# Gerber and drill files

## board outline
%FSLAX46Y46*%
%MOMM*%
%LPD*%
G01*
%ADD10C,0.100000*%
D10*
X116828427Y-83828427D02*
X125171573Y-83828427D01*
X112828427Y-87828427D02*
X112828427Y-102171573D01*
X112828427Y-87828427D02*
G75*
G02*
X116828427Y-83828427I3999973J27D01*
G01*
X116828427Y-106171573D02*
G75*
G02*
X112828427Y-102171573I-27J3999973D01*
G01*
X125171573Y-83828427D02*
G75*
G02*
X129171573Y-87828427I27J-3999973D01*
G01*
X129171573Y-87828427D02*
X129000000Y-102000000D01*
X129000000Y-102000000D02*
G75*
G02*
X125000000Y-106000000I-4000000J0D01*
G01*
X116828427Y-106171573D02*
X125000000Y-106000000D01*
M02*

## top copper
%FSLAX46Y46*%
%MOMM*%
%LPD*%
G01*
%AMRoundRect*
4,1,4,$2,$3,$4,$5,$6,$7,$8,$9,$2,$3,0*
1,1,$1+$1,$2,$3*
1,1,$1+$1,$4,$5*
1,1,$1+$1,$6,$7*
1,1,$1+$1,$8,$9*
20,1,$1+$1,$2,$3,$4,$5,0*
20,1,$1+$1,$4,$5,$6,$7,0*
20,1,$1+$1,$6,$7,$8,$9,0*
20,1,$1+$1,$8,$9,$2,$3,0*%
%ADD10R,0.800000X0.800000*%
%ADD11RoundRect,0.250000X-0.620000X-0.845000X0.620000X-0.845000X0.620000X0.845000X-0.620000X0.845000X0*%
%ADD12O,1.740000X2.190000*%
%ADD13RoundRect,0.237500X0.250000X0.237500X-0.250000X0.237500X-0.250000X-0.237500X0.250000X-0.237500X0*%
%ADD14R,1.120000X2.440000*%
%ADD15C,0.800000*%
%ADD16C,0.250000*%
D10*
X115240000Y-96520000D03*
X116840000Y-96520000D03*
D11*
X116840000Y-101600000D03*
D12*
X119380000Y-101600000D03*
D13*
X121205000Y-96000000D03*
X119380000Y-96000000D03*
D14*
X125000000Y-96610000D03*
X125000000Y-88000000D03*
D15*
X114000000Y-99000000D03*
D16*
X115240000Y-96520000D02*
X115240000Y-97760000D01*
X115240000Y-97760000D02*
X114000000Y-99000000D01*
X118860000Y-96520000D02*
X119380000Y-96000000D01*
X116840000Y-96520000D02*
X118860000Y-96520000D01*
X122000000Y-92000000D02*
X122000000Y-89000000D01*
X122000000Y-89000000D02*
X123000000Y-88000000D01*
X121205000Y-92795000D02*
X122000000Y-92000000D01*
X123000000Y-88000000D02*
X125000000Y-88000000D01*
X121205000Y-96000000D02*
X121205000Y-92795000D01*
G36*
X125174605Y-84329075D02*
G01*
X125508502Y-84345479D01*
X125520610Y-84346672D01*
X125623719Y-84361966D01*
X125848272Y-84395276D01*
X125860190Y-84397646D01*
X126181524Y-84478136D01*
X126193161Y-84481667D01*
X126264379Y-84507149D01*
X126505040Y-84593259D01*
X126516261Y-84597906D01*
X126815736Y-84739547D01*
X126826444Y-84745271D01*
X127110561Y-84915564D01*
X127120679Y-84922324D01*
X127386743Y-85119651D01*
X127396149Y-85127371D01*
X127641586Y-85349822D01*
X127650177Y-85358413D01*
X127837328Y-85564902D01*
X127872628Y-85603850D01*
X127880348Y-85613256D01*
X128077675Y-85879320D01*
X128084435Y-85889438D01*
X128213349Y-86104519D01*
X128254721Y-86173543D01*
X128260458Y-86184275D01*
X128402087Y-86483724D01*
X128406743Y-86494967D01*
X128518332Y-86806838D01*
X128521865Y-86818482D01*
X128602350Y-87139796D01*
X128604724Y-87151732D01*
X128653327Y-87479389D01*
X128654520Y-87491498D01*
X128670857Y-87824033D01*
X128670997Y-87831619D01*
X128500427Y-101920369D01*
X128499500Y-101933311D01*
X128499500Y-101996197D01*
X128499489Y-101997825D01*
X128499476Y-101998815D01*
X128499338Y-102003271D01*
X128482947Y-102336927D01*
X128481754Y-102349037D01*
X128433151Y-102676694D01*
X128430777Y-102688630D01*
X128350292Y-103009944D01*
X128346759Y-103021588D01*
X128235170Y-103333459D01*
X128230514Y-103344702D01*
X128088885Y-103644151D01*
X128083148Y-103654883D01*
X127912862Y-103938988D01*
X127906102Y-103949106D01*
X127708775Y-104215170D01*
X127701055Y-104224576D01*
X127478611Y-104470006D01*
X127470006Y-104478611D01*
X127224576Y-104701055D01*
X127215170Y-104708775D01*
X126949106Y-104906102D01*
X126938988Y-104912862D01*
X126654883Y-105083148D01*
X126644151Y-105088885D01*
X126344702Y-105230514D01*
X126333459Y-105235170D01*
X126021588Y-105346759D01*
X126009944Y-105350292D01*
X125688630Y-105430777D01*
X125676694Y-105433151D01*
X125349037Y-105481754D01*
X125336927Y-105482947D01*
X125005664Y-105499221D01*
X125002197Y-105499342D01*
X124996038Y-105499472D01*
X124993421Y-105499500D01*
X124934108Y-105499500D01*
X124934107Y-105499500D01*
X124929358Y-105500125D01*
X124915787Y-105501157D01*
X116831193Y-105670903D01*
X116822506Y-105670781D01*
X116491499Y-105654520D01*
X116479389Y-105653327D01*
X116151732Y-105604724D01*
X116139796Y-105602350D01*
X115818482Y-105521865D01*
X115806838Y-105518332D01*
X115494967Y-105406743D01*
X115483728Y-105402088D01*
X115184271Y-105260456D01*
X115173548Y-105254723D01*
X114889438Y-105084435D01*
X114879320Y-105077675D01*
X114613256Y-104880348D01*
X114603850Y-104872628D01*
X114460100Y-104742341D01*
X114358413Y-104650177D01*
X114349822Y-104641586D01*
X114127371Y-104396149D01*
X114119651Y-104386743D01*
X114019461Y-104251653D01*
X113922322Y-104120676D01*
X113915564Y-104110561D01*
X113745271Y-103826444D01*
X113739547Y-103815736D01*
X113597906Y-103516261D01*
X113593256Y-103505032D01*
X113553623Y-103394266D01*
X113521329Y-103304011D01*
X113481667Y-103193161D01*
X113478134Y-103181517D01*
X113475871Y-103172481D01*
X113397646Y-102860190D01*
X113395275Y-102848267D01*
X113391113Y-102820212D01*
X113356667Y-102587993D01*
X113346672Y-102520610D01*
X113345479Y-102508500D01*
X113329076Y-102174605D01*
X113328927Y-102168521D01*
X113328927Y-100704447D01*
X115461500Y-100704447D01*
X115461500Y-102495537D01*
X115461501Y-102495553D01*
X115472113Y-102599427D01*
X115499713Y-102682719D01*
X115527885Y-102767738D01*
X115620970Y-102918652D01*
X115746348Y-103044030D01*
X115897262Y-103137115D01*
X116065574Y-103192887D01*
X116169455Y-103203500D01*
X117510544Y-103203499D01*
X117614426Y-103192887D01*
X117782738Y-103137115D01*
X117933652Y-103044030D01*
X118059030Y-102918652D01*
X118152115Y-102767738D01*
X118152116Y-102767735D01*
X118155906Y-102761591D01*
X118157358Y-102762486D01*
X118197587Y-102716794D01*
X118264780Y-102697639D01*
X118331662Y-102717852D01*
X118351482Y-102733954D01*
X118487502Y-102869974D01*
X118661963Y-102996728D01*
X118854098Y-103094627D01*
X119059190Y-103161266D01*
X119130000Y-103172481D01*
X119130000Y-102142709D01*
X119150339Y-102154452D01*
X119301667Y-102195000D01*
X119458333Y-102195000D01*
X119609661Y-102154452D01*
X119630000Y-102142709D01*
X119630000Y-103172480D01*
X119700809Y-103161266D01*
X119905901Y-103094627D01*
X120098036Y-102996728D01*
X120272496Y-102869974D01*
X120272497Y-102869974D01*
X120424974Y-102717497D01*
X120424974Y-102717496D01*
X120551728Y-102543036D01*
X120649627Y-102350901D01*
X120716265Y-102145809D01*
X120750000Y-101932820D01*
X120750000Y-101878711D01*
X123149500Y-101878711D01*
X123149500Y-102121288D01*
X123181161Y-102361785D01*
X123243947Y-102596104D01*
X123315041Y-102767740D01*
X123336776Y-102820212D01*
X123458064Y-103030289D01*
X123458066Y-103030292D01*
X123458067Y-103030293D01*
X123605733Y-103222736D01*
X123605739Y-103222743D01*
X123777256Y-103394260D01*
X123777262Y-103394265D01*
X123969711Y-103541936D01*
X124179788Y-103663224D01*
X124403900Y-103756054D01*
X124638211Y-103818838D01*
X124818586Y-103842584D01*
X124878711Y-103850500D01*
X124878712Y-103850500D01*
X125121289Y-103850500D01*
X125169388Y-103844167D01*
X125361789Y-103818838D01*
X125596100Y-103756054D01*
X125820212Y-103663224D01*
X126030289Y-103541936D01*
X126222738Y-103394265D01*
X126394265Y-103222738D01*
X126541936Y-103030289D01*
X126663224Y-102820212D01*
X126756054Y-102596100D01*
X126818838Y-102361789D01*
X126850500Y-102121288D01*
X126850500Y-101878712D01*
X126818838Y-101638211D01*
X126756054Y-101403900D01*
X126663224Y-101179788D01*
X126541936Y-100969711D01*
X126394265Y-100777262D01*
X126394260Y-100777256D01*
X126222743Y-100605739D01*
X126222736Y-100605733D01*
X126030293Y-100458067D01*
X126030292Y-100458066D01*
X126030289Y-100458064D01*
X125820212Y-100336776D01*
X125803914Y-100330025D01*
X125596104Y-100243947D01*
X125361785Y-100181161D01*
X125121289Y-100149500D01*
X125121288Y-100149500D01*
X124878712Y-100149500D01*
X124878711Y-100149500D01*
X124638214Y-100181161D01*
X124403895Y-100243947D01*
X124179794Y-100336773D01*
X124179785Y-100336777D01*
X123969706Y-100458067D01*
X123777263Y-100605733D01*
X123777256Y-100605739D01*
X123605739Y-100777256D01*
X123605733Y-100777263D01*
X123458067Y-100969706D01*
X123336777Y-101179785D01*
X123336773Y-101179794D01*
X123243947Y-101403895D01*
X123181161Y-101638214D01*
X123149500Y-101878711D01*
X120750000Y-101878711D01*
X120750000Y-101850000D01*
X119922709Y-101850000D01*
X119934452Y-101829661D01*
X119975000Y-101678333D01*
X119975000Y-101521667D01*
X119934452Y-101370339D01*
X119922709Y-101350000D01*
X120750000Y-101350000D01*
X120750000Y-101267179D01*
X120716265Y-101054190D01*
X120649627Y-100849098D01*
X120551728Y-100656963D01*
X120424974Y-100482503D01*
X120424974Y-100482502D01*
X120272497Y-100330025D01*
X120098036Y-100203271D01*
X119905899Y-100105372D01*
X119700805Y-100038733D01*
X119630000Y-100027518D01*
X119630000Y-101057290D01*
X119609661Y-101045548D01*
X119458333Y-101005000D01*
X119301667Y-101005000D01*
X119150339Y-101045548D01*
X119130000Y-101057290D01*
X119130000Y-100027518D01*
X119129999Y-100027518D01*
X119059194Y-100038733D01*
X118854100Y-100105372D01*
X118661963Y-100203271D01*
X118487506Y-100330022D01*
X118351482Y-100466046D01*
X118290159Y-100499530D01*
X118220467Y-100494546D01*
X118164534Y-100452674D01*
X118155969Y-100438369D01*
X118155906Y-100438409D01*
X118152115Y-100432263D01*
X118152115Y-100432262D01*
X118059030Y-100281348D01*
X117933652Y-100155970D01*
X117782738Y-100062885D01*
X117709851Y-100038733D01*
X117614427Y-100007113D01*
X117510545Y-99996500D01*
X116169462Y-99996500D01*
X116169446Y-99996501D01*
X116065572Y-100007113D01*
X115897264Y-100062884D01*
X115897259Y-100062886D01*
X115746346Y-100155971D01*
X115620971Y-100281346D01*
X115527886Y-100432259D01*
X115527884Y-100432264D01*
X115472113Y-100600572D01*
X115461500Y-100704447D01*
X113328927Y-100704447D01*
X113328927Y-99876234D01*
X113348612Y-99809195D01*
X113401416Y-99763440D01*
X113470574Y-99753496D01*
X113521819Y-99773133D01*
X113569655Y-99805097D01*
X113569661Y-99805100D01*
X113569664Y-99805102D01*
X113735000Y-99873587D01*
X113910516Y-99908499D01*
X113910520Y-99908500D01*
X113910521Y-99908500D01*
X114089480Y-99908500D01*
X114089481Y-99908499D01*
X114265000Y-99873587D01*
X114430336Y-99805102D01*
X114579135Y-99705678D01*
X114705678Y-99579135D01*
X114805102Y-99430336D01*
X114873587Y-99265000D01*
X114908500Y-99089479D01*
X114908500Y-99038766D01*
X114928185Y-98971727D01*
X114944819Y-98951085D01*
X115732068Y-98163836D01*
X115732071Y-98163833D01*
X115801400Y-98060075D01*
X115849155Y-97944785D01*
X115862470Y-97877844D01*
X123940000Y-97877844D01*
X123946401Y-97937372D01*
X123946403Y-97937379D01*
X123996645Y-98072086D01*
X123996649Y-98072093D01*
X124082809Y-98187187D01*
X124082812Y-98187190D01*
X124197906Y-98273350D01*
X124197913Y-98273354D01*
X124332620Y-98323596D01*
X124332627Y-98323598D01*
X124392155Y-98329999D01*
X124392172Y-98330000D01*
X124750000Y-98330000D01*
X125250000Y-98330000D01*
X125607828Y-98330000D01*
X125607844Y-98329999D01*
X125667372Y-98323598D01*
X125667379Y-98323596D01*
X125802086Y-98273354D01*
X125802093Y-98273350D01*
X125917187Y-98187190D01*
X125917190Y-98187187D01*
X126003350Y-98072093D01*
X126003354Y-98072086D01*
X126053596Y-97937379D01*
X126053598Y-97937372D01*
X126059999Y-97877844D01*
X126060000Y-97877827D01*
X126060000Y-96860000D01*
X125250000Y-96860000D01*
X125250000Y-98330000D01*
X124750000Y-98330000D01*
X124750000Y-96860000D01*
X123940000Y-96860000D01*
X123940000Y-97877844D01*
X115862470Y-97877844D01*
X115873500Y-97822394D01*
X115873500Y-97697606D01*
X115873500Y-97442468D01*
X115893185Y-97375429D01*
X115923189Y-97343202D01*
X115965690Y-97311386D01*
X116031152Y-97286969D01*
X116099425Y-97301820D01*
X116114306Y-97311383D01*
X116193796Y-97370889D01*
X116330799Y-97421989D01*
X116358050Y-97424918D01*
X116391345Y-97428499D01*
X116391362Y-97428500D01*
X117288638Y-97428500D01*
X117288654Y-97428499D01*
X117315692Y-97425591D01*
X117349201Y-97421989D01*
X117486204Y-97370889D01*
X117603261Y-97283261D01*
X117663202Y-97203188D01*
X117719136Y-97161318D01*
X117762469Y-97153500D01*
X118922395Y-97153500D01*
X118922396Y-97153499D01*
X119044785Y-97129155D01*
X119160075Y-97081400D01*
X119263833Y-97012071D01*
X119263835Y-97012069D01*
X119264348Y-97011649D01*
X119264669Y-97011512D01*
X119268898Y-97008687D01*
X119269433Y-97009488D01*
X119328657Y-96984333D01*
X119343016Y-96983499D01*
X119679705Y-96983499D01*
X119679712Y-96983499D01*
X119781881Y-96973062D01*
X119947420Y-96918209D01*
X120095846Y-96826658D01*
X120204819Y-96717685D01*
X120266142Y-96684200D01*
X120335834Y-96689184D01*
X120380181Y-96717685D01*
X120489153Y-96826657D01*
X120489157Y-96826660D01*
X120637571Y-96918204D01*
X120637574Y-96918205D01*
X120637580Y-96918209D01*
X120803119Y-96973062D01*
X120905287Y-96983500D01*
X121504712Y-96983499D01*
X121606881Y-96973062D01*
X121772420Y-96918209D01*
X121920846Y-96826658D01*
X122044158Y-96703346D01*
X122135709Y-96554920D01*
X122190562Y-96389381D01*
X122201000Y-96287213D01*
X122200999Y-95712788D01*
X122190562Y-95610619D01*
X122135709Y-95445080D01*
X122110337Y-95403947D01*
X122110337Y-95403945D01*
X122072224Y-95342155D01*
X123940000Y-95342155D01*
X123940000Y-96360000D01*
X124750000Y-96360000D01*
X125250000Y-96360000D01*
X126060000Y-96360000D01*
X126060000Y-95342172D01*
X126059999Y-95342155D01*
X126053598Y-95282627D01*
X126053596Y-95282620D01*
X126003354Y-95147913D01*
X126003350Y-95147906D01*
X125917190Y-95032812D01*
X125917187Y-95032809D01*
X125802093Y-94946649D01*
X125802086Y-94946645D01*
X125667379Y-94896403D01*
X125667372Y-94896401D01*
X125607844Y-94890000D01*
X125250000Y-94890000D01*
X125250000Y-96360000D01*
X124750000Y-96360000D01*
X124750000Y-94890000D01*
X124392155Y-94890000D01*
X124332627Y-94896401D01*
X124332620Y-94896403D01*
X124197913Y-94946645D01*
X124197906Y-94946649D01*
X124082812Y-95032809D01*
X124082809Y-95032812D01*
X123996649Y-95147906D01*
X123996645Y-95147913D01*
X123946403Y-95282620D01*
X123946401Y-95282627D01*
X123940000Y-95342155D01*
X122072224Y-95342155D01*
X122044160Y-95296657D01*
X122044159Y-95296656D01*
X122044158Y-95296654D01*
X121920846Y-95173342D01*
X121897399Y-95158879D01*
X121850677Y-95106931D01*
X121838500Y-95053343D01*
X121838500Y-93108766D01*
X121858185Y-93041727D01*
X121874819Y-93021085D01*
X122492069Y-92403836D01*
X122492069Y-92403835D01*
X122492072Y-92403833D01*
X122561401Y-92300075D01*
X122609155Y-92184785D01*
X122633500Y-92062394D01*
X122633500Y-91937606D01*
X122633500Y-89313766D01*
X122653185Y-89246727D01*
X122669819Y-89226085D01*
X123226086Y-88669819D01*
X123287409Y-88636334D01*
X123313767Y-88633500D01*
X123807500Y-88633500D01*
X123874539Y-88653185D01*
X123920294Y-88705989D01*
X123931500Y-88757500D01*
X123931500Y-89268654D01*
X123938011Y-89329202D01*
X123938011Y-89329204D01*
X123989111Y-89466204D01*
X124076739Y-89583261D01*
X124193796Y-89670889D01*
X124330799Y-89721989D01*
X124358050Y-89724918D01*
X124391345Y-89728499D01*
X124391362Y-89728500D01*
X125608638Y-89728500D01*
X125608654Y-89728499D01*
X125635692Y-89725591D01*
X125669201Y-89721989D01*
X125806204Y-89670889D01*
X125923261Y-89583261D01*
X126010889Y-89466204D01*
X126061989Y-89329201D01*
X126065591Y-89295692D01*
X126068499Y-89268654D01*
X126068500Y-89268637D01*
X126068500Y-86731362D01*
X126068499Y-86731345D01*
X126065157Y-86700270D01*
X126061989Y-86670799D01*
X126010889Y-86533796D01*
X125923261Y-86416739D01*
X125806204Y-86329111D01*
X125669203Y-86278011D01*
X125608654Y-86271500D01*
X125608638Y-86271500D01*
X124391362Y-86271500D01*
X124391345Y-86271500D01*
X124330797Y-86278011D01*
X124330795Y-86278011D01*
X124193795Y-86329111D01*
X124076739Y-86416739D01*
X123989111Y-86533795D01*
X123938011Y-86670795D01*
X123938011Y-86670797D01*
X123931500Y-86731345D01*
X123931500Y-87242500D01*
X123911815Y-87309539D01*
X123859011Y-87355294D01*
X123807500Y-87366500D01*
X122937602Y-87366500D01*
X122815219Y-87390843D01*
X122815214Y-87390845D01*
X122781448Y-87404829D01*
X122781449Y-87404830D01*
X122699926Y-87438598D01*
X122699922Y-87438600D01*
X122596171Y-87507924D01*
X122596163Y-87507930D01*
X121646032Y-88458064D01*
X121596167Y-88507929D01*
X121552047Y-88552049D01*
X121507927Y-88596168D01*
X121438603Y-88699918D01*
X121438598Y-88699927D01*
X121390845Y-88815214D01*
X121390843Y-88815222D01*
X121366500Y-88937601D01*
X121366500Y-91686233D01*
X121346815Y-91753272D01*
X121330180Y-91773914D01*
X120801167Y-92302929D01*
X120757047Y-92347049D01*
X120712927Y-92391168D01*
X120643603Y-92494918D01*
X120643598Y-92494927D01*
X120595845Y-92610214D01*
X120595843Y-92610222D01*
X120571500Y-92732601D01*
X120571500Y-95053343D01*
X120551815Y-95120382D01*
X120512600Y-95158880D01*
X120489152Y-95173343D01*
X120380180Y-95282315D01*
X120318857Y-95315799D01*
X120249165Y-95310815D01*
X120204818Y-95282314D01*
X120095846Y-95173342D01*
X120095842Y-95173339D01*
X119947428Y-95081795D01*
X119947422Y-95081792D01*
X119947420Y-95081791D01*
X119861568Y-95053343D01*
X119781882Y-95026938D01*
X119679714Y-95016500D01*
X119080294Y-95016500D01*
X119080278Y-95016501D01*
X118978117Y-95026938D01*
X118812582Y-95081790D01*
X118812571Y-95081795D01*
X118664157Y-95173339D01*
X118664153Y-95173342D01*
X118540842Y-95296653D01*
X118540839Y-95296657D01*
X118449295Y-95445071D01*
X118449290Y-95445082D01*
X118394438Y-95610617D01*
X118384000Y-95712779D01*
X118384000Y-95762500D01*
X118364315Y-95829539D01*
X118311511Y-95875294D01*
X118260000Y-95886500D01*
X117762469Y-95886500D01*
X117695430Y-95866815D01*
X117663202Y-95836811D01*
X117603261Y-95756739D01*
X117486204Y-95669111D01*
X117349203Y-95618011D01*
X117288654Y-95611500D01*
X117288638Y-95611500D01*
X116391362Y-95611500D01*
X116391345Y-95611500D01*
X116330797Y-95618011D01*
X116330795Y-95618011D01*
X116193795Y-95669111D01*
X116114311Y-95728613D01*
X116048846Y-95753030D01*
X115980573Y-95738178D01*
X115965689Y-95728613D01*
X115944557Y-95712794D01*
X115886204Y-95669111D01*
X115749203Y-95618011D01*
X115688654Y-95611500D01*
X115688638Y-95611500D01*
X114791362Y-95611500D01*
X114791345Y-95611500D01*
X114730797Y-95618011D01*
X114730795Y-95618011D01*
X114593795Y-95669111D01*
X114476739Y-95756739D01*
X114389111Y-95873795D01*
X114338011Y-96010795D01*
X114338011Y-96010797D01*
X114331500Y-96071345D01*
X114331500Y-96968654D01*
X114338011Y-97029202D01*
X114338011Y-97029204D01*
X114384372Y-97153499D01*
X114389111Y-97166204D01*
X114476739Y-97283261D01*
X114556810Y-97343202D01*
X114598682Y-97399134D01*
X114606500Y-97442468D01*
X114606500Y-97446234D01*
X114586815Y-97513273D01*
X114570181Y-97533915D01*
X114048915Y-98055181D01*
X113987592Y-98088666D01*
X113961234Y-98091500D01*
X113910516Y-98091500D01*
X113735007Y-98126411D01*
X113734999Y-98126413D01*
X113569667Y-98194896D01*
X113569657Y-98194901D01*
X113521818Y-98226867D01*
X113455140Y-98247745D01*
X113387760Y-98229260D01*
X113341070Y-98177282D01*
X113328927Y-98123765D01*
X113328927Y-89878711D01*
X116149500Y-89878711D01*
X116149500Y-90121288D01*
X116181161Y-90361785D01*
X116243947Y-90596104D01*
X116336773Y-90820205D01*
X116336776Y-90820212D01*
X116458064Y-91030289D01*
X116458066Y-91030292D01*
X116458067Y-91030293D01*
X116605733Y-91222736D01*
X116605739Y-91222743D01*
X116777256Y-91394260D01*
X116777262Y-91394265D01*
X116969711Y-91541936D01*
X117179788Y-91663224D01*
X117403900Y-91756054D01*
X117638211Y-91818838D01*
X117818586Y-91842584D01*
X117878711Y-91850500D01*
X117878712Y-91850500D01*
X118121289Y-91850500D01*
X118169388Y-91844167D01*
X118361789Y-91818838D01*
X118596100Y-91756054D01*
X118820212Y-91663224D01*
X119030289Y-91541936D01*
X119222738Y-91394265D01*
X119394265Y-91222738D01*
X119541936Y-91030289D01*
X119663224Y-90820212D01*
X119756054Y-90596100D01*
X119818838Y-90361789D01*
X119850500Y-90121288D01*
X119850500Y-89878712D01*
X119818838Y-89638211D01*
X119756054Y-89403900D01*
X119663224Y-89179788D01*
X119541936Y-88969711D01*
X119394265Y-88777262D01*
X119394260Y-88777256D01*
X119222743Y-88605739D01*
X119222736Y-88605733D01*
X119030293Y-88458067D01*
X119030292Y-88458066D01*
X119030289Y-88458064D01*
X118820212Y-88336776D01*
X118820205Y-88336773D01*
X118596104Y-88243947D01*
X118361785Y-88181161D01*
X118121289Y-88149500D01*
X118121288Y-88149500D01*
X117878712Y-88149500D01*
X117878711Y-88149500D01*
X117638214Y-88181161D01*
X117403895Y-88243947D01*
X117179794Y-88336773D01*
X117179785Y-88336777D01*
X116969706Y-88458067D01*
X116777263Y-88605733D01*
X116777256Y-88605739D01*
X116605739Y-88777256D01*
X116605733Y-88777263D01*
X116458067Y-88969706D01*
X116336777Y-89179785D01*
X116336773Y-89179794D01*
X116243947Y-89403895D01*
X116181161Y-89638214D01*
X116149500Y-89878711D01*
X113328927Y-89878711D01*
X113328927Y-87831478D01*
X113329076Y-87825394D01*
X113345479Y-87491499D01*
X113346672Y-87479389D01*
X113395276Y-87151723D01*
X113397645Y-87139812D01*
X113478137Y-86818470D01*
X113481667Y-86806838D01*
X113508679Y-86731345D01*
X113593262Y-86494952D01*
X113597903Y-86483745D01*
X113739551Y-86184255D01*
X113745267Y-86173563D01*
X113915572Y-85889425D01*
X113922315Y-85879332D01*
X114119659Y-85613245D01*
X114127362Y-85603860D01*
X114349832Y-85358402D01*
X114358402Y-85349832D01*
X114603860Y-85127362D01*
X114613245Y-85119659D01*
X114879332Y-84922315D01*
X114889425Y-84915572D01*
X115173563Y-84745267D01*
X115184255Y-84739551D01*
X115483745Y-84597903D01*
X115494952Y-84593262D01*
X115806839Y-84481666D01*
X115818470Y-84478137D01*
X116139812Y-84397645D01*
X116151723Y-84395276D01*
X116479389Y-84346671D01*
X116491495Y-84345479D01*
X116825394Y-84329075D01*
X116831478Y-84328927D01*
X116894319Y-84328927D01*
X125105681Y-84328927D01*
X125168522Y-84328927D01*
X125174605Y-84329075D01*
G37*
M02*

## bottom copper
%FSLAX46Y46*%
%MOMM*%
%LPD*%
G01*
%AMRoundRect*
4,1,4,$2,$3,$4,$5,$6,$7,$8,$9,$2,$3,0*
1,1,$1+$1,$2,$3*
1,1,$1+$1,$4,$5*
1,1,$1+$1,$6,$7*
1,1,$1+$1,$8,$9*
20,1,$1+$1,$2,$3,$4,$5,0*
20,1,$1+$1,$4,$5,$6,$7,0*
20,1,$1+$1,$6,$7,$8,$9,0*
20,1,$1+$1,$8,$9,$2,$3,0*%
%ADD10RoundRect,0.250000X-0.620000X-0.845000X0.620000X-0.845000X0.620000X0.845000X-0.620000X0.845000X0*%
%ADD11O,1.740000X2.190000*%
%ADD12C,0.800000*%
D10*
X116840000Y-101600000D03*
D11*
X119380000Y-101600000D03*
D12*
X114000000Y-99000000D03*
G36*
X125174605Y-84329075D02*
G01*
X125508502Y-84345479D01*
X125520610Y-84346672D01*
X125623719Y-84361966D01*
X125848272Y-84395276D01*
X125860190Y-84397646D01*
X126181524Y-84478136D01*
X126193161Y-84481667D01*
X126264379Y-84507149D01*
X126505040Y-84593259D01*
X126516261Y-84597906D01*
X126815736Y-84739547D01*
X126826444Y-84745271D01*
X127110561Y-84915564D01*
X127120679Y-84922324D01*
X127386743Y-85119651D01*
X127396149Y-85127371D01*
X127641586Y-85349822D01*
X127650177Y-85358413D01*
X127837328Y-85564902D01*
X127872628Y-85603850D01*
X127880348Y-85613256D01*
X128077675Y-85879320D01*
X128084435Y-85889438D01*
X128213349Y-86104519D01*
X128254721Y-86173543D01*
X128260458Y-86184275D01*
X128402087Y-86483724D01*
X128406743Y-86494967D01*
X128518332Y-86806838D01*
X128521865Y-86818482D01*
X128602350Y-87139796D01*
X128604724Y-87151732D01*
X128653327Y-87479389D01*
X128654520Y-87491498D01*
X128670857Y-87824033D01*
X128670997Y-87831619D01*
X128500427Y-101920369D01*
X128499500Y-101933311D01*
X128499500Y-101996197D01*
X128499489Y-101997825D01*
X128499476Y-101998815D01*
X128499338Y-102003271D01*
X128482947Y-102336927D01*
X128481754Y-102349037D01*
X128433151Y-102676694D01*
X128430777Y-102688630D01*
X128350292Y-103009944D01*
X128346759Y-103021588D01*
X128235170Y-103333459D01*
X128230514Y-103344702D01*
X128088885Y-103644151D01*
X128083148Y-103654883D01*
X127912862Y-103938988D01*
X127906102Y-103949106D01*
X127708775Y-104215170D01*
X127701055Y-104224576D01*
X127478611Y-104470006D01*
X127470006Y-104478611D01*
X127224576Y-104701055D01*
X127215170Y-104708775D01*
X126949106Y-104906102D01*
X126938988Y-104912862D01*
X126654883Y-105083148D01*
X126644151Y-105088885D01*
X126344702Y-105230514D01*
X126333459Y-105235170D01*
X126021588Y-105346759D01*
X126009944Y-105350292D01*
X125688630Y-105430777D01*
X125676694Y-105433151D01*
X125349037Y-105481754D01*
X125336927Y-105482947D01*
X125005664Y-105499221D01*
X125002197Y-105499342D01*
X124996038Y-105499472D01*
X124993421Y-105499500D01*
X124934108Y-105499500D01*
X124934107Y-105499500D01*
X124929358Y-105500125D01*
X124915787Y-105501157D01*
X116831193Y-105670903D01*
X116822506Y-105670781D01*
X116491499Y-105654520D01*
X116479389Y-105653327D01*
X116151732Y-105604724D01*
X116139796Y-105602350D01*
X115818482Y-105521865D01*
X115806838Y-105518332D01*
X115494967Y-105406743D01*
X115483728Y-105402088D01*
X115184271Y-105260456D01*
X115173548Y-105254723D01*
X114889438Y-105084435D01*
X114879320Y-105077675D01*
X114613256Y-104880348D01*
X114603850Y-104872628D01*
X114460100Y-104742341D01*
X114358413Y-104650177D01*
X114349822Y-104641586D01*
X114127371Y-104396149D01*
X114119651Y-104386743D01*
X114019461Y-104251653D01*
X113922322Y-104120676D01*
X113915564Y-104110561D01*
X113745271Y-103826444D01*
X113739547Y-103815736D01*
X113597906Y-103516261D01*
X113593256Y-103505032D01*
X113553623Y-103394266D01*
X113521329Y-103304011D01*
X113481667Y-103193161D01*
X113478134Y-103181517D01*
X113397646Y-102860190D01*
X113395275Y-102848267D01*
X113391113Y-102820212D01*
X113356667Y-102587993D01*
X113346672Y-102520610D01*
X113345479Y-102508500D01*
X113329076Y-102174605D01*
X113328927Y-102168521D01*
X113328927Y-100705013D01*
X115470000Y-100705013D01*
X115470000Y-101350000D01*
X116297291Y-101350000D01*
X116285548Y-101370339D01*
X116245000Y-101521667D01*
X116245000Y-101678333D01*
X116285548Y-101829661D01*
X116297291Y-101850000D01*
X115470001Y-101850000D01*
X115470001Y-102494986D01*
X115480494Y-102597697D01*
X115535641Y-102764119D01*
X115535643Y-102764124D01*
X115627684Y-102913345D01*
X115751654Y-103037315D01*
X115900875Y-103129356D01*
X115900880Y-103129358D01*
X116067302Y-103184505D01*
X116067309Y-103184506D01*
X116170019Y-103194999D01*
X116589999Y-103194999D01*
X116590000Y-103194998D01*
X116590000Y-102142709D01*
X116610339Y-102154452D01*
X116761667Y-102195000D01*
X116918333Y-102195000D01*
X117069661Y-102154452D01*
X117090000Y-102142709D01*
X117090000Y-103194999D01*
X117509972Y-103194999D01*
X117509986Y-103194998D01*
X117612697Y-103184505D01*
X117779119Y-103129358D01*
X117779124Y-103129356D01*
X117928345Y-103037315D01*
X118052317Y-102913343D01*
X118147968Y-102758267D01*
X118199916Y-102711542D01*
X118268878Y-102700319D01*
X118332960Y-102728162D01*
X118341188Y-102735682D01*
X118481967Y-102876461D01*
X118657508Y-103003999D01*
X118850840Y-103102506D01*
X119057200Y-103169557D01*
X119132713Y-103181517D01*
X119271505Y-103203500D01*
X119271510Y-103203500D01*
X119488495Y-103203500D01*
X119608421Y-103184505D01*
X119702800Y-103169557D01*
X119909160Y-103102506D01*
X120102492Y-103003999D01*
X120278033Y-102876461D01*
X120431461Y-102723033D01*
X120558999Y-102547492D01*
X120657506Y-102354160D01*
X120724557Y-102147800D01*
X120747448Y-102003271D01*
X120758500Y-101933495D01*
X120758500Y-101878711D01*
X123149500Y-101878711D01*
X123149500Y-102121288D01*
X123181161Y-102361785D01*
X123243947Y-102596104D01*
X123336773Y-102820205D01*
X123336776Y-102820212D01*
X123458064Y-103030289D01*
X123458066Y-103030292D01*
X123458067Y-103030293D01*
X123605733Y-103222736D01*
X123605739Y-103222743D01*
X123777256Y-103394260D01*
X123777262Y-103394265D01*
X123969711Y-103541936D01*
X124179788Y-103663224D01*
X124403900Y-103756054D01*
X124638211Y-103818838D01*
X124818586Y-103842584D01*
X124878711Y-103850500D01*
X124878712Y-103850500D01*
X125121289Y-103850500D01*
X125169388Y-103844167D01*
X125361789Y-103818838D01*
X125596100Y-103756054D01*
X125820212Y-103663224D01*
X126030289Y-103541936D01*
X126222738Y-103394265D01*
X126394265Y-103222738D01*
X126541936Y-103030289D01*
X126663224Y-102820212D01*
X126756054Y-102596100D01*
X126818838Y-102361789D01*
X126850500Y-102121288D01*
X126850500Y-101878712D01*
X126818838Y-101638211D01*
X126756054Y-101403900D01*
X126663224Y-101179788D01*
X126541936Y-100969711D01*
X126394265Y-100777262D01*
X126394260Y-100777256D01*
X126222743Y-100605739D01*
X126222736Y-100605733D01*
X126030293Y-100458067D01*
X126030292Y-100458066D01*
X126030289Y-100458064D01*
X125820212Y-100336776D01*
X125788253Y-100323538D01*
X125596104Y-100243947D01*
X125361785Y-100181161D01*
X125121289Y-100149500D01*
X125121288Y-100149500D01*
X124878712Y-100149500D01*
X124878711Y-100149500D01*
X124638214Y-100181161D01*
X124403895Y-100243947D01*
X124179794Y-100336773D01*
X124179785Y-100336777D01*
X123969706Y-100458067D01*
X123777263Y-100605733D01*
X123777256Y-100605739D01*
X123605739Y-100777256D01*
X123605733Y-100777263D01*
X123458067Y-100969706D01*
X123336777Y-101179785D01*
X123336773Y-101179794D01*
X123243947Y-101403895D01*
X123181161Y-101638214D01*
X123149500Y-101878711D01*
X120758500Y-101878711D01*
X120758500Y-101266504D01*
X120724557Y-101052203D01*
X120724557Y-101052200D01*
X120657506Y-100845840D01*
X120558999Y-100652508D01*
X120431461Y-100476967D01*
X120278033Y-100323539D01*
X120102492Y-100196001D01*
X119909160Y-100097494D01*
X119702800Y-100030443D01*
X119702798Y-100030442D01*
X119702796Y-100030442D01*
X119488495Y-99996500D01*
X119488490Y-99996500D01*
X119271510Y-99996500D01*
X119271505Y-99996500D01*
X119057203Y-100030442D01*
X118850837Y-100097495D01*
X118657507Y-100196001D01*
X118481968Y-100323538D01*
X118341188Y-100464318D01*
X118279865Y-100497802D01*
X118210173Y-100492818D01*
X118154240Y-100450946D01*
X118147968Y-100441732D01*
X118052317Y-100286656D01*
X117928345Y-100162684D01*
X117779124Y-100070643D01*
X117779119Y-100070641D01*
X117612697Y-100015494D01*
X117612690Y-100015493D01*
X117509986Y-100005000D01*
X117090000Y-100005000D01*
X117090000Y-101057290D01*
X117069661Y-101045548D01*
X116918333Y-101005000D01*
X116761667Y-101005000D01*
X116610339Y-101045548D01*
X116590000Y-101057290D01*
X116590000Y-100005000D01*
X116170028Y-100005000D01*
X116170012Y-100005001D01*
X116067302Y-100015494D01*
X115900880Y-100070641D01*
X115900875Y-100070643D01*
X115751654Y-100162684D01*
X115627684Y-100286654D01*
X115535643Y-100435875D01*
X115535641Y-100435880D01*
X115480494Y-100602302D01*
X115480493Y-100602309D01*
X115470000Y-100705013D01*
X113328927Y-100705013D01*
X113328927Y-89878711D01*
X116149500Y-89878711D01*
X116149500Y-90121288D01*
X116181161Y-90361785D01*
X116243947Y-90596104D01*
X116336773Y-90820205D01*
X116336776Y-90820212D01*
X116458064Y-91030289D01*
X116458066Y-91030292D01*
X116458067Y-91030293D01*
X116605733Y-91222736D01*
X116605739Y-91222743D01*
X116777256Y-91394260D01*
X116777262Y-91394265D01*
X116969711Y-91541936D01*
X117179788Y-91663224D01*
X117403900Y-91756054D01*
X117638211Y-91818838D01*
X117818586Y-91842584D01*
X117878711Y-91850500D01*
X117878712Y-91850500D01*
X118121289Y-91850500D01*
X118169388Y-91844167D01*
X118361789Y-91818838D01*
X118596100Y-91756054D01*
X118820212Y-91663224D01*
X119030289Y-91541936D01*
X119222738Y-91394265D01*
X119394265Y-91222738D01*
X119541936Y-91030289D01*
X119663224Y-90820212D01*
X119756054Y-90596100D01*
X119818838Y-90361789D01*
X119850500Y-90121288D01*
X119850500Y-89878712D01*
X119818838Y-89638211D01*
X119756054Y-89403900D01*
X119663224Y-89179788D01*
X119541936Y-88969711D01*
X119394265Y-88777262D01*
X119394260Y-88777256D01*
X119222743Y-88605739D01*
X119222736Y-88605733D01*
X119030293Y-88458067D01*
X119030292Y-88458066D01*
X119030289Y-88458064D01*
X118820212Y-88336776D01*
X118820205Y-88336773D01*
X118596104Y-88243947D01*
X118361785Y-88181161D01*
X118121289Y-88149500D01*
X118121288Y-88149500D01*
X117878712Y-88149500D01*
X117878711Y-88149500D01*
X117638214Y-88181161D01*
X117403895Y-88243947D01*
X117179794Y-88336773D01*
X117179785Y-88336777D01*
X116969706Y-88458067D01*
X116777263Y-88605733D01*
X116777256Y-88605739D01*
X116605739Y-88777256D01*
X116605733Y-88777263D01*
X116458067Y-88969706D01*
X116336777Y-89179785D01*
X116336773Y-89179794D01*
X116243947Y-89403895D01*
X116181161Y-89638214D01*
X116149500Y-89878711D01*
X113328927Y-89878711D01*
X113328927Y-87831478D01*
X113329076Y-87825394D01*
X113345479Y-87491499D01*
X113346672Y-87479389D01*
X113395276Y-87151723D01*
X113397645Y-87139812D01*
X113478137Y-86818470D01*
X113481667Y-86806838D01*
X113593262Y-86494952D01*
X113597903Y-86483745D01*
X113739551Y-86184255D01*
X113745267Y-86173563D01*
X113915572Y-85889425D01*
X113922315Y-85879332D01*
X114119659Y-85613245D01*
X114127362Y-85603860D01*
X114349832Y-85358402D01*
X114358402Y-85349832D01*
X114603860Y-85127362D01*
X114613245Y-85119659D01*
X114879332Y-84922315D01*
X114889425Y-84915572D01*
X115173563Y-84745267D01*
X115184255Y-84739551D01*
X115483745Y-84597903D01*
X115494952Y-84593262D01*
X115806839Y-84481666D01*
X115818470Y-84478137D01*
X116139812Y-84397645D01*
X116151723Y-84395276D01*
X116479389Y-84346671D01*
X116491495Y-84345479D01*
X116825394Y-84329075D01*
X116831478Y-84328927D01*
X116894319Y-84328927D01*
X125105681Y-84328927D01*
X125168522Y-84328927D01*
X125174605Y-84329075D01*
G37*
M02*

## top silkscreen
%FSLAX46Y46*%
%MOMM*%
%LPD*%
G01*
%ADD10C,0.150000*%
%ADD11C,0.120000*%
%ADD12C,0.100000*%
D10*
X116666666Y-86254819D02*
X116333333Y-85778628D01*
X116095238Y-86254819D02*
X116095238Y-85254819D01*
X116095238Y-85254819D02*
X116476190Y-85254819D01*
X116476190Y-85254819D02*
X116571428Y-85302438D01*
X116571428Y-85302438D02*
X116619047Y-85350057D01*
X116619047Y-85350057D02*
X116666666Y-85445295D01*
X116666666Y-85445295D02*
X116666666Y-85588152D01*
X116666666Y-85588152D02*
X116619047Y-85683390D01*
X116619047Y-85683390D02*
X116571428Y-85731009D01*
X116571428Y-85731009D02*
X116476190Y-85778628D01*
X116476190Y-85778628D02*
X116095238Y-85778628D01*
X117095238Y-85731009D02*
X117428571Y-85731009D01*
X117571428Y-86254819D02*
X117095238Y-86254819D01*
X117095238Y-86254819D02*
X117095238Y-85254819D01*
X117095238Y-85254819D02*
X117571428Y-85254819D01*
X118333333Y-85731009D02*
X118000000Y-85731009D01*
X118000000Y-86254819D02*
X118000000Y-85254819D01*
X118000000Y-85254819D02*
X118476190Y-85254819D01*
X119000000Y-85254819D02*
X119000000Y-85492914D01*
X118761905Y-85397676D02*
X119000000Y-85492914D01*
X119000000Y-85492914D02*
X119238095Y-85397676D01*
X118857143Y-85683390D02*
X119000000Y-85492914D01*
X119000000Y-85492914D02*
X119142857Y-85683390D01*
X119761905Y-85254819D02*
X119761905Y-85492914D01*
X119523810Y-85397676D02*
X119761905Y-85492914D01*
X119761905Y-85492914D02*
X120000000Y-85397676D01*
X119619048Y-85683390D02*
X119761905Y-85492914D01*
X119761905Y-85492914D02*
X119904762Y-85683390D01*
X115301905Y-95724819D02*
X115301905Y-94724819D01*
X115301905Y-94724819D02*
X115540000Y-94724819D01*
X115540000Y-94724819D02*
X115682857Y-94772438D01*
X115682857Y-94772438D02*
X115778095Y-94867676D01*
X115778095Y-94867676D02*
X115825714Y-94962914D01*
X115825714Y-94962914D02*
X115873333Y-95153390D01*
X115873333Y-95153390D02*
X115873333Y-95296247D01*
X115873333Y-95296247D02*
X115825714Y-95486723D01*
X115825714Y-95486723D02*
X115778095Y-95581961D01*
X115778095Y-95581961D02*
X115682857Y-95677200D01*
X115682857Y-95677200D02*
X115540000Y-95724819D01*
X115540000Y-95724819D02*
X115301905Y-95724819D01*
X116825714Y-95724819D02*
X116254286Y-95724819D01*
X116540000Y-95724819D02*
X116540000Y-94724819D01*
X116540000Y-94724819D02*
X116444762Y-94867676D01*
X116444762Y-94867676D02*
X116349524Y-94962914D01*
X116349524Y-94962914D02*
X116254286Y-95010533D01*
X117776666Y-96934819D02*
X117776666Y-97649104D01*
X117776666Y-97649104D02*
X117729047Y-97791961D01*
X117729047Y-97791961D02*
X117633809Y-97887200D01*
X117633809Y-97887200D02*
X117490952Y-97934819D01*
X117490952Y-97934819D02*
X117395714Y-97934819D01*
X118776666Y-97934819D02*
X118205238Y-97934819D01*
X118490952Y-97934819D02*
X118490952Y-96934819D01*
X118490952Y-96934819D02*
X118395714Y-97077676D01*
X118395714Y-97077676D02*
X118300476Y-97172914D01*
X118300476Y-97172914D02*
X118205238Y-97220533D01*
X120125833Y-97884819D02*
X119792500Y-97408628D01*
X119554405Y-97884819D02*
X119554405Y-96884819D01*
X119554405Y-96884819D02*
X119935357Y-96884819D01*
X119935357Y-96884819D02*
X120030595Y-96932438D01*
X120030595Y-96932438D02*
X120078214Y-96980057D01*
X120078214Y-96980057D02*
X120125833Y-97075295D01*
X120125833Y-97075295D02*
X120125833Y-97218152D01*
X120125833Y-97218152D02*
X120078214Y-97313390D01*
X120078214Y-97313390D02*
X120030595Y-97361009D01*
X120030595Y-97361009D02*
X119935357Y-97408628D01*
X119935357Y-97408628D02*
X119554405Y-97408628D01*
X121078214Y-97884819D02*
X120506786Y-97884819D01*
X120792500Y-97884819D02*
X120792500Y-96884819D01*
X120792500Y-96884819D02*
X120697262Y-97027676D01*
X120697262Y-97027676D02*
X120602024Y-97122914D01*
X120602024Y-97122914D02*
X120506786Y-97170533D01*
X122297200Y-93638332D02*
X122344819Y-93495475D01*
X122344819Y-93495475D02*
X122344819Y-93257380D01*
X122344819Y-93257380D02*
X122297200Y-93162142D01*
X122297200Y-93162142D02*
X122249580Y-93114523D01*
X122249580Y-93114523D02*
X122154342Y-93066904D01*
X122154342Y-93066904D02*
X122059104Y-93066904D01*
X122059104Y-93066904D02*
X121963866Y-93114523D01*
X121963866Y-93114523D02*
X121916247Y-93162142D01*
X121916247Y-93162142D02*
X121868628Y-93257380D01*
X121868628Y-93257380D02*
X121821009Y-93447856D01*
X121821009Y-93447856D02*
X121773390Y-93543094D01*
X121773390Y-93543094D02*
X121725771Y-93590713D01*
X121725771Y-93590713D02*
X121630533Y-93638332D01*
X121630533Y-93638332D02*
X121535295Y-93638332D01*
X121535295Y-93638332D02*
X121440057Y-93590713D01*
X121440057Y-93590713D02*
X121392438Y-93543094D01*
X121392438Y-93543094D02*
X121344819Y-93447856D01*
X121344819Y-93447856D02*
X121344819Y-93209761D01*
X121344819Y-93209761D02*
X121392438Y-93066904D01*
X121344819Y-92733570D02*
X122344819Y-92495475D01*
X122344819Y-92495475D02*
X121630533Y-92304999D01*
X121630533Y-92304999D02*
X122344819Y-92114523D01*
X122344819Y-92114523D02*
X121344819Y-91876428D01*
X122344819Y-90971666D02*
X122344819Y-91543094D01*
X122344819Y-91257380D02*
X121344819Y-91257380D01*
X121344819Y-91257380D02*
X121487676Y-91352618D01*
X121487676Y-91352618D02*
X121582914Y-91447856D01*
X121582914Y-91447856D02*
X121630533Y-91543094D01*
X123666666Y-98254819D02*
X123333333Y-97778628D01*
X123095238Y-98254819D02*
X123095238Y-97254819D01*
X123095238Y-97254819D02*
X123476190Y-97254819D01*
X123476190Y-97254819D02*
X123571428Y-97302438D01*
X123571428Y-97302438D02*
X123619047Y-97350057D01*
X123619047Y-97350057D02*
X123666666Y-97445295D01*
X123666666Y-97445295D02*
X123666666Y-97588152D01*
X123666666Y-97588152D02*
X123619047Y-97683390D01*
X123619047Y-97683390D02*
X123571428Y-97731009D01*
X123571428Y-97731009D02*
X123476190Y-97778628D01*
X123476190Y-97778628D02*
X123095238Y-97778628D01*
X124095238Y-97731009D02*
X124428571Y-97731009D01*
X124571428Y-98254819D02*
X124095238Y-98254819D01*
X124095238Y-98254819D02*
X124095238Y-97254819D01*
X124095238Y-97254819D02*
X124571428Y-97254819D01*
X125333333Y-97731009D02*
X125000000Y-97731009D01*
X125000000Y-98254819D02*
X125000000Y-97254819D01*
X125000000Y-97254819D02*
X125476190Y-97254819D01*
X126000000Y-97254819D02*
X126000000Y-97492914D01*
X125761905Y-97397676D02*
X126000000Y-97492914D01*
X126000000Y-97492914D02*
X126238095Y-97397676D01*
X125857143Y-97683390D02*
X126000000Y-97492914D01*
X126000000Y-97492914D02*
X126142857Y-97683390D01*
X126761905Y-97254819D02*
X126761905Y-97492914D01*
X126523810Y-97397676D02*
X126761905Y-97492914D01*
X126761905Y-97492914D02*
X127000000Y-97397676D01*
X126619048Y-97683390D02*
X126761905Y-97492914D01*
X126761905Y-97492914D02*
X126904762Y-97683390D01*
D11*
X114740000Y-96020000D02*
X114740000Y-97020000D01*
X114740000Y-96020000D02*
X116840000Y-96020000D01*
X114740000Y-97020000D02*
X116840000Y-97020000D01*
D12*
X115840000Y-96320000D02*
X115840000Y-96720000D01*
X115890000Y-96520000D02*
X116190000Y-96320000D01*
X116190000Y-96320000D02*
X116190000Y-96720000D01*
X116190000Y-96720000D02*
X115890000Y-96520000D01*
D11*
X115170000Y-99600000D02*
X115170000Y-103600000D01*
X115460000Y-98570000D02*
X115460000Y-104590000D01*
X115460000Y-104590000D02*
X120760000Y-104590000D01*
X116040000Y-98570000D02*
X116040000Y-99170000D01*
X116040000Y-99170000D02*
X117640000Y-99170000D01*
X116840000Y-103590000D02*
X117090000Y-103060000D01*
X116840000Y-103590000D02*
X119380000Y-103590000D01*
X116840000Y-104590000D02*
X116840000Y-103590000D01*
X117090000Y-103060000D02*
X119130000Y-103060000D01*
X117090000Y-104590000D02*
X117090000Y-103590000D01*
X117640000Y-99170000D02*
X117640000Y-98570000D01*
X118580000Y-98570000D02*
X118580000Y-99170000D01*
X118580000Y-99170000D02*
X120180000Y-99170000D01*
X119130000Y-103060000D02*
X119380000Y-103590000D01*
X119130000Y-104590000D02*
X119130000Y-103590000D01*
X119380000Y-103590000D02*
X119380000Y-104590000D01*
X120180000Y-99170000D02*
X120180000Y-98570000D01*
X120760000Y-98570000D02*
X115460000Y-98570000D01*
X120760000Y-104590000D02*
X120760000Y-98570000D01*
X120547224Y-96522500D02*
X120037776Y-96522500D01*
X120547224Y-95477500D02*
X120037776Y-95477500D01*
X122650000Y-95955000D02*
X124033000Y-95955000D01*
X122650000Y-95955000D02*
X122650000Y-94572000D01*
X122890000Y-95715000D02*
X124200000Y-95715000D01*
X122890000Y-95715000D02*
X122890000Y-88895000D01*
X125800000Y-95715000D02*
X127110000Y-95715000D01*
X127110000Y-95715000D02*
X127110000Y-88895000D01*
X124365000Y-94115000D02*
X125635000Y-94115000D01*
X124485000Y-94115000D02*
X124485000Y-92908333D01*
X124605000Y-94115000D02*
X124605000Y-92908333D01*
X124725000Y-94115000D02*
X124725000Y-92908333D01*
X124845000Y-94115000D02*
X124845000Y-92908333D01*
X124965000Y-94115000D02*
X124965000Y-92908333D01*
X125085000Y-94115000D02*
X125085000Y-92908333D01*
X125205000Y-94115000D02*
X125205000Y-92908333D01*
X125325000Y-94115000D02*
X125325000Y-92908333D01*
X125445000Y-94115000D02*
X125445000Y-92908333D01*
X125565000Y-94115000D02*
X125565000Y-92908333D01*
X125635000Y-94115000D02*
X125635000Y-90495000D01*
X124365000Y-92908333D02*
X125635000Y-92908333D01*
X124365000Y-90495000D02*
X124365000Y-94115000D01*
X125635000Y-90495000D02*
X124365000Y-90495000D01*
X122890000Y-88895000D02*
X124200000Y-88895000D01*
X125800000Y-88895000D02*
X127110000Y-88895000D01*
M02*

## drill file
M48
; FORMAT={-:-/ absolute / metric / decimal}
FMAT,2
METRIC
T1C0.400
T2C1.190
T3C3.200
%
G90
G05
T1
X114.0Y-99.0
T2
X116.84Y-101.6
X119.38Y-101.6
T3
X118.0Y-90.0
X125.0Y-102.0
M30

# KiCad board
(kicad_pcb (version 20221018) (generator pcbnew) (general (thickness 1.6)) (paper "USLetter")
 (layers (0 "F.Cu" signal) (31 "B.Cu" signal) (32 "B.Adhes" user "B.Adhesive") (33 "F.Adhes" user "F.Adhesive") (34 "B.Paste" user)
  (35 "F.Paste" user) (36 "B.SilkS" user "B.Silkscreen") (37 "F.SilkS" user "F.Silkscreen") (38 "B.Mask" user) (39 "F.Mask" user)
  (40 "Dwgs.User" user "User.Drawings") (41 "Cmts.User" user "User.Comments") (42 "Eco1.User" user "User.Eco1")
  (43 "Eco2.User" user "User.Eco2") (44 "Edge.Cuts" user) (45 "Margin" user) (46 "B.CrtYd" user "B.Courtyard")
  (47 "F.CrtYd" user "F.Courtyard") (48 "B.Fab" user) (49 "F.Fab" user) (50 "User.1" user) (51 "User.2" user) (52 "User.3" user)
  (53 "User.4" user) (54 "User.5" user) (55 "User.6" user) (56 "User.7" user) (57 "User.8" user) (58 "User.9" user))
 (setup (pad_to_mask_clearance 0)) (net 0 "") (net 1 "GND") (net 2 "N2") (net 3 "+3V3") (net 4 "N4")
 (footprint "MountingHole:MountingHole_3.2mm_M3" (layer "F.Cu") (at 118 90)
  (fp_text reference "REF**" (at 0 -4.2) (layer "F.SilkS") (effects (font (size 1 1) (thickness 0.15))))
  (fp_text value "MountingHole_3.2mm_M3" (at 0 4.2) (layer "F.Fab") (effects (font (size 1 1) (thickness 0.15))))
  (pad "" np_thru_hole circle (at 0 0) (size 3.2 3.2) (drill 3.2) (layers "*.Cu" "*.Mask")))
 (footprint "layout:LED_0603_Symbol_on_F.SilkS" (layer "F.Cu") (at 116.04 96.52)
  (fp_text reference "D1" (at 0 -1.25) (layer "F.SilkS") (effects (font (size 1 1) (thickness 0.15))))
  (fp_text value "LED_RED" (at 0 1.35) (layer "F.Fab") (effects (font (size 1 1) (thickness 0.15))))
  (fp_line (start -1.3 -0.5) (end -1.3 0.5) (stroke (width 0.12) (type solid)) (layer "F.SilkS"))
  (fp_line (start -1.3 -0.5) (end 0.8 -0.5) (stroke (width 0.12) (type solid)) (layer "F.SilkS"))
  (fp_line (start -1.3 0.5) (end 0.8 0.5) (stroke (width 0.12) (type solid)) (layer "F.SilkS"))
  (fp_line (start -0.2 -0.2) (end -0.2 0.2) (stroke (width 0.1) (type solid)) (layer "F.SilkS"))
  (fp_line (start -0.15 0) (end 0.15 -0.2) (stroke (width 0.1) (type solid)) (layer "F.SilkS"))
  (fp_line (start 0.15 -0.2) (end 0.15 0.2) (stroke (width 0.1) (type solid)) (layer "F.SilkS"))
  (fp_line (start 0.15 0.2) (end -0.15 0) (stroke (width 0.1) (type solid)) (layer "F.SilkS"))
  (pad "1" smd rect (at -0.8 0 180) (size 0.8 0.8) (layers "F.Cu" "F.Paste" "F.Mask") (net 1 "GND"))
  (pad "2" smd rect (at 0.8 0 180) (size 0.8 0.8) (layers "F.Cu" "F.Paste" "F.Mask") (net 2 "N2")))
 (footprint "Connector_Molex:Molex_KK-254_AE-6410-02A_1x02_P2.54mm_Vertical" (layer "F.Cu") (at 116.84 101.6)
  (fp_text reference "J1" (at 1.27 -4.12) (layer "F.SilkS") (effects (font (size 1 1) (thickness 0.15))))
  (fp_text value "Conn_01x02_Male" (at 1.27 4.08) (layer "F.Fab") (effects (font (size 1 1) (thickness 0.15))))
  (fp_line (start -1.67 -2) (end -1.67 2) (stroke (width 0.12) (type solid)) (layer "F.SilkS"))
  (fp_line (start -1.38 -3.03) (end -1.38 2.99) (stroke (width 0.12) (type solid)) (layer "F.SilkS"))
  (fp_line (start -1.38 2.99) (end 3.92 2.99) (stroke (width 0.12) (type solid)) (layer "F.SilkS"))
  (fp_line (start -0.8 -3.03) (end -0.8 -2.43) (stroke (width 0.12) (type solid)) (layer "F.SilkS"))
  (fp_line (start -0.8 -2.43) (end 0.8 -2.43) (stroke (width 0.12) (type solid)) (layer "F.SilkS"))
  (fp_line (start 0 1.99) (end 0.25 1.46) (stroke (width 0.12) (type solid)) (layer "F.SilkS"))
  (fp_line (start 0 1.99) (end 2.54 1.99) (stroke (width 0.12) (type solid)) (layer "F.SilkS"))
  (fp_line (start 0 2.99) (end 0 1.99) (stroke (width 0.12) (type solid)) (layer "F.SilkS"))
  (fp_line (start 0.25 1.46) (end 2.29 1.46) (stroke (width 0.12) (type solid)) (layer "F.SilkS"))
  (fp_line (start 0.25 2.99) (end 0.25 1.99) (stroke (width 0.12) (type solid)) (layer "F.SilkS"))
  (fp_line (start 0.8 -2.43) (end 0.8 -3.03) (stroke (width 0.12) (type solid)) (layer "F.SilkS"))
  (fp_line (start 1.74 -3.03) (end 1.74 -2.43) (stroke (width 0.12) (type solid)) (layer "F.SilkS"))
  (fp_line (start 1.74 -2.43) (end 3.34 -2.43) (stroke (width 0.12) (type solid)) (layer "F.SilkS"))
  (fp_line (start 2.29 1.46) (end 2.54 1.99) (stroke (width 0.12) (type solid)) (layer "F.SilkS"))
  (fp_line (start 2.29 2.99) (end 2.29 1.99) (stroke (width 0.12) (type solid)) (layer "F.SilkS"))
  (fp_line (start 2.54 1.99) (end 2.54 2.99) (stroke (width 0.12) (type solid)) (layer "F.SilkS"))
  (fp_line (start 3.34 -2.43) (end 3.34 -3.03) (stroke (width 0.12) (type solid)) (layer "F.SilkS"))
  (fp_line (start 3.92 -3.03) (end -1.38 -3.03) (stroke (width 0.12) (type solid)) (layer "F.SilkS"))
  (fp_line (start 3.92 2.99) (end 3.92 -3.03) (stroke (width 0.12) (type solid)) (layer "F.SilkS"))
  (pad "1" thru_hole roundrect (at 0 0) (size 1.74 2.19) (drill 1.19) (layers "*.Cu" "*.Mask") (roundrect_rratio 0.143678) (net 1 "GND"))
  (pad "2" thru_hole oval (at 2.54 0) (size 1.74 2.19) (drill 1.19) (layers "*.Cu" "*.Mask") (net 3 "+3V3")))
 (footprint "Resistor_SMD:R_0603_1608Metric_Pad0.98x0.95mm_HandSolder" (layer "F.Cu") (at 120.2925 96 180)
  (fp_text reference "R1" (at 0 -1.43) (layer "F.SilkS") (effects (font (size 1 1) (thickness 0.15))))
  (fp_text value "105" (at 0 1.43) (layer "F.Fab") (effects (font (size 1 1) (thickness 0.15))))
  (fp_line (start -0.254724 -0.5225) (end 0.254724 -0.5225) (stroke (width 0.12) (type solid)) (layer "F.SilkS"))
  (fp_line (start -0.254724 0.5225) (end 0.254724 0.5225) (stroke (width 0.12) (type solid)) (layer "F.SilkS"))
  (pad "1" smd roundrect (at -0.9125 0 180) (size 0.975 0.95) (layers "F.Cu" "F.Paste" "F.Mask") (roundrect_rratio 0.25) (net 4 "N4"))
  (pad "2" smd roundrect (at 0.9125 0 180) (size 0.975 0.95) (layers "F.Cu" "F.Paste" "F.Mask") (roundrect_rratio 0.25) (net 2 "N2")))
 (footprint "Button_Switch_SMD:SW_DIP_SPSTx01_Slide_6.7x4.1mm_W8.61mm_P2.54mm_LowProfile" (layer "F.Cu") (at 125 92.305 90)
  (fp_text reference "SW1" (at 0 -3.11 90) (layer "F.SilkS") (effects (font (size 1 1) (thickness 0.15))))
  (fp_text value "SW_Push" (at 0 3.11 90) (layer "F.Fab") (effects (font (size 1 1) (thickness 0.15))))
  (fp_line (start -3.65 -2.35) (end -3.65 -0.967) (stroke (width 0.12) (type solid)) (layer "F.SilkS"))
  (fp_line (start -3.65 -2.35) (end -2.267 -2.35) (stroke (width 0.12) (type solid)) (layer "F.SilkS"))
  (fp_line (start -3.41 -2.11) (end -3.41 -0.8) (stroke (width 0.12) (type solid)) (layer "F.SilkS"))
  (fp_line (start -3.41 -2.11) (end 3.41 -2.11) (stroke (width 0.12) (type solid)) (layer "F.SilkS"))
  (fp_line (start -3.41 0.8) (end -3.41 2.11) (stroke (width 0.12) (type solid)) (layer "F.SilkS"))
  (fp_line (start -3.41 2.11) (end 3.41 2.11) (stroke (width 0.12) (type solid)) (layer "F.SilkS"))
  (fp_line (start -1.81 -0.635) (end -1.81 0.635) (stroke (width 0.12) (type solid)) (layer "F.SilkS"))
  (fp_line (start -1.81 -0.515) (end -0.603333 -0.515) (stroke (width 0.12) (type solid)) (layer "F.SilkS"))
  (fp_line (start -1.81 -0.395) (end -0.603333 -0.395) (stroke (width 0.12) (type solid)) (layer "F.SilkS"))
  (fp_line (start -1.81 -0.275) (end -0.603333 -0.275) (stroke (width 0.12) (type solid)) (layer "F.SilkS"))
  (fp_line (start -1.81 -0.155) (end -0.603333 -0.155) (stroke (width 0.12) (type solid)) (layer "F.SilkS"))
  (fp_line (start -1.81 -0.035) (end -0.603333 -0.035) (stroke (width 0.12) (type solid)) (layer "F.SilkS"))
  (fp_line (start -1.81 0.085) (end -0.603333 0.085) (stroke (width 0.12) (type solid)) (layer "F.SilkS"))
  (fp_line (start -1.81 0.205) (end -0.603333 0.205) (stroke (width 0.12) (type solid)) (layer "F.SilkS"))
  (fp_line (start -1.81 0.325) (end -0.603333 0.325) (stroke (width 0.12) (type solid)) (layer "F.SilkS"))
  (fp_line (start -1.81 0.445) (end -0.603333 0.445) (stroke (width 0.12) (type solid)) (layer "F.SilkS"))
  (fp_line (start -1.81 0.565) (end -0.603333 0.565) (stroke (width 0.12) (type solid)) (layer "F.SilkS"))
  (fp_line (start -1.81 0.635) (end 1.81 0.635) (stroke (width 0.12) (type solid)) (layer "F.SilkS"))
  (fp_line (start -0.603333 -0.635) (end -0.603333 0.635) (stroke (width 0.12) (type solid)) (layer "F.SilkS"))
  (fp_line (start 1.81 -0.635) (end -1.81 -0.635) (stroke (width 0.12) (type solid)) (layer "F.SilkS"))
  (fp_line (start 1.81 0.635) (end 1.81 -0.635) (stroke (width 0.12) (type solid)) (layer "F.SilkS"))
  (fp_line (start 3.41 -2.11) (end 3.41 -0.8) (stroke (width 0.12) (type solid)) (layer "F.SilkS"))
  (fp_line (start 3.41 0.8) (end 3.41 2.11) (stroke (width 0.12) (type solid)) (layer "F.SilkS"))
  (pad "1" smd rect (at -4.305 0 90) (size 2.44 1.12) (layers "F.Cu" "F.Paste" "F.Mask") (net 3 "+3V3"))
  (pad "2" smd rect (at 4.305 0 90) (size 2.44 1.12) (layers "F.Cu" "F.Paste" "F.Mask") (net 4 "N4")))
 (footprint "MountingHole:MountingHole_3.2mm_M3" (layer "F.Cu") (at 125 102)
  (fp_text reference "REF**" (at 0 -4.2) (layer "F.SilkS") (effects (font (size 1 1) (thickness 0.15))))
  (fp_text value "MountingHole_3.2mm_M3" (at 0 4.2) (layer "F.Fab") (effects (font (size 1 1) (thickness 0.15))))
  (pad "" np_thru_hole circle (at 0 0) (size 3.2 3.2) (drill 3.2) (layers "*.Cu" "*.Mask")))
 (gr_line (start 116.828427 83.828427) (end 125.171573 83.828427) (stroke (width 0.1) (type default)) (layer "Edge.Cuts"))
 (gr_line (start 112.828427 87.828427) (end 112.828427 102.171573) (stroke (width 0.1) (type default)) (layer "Edge.Cuts"))
 (gr_arc (start 112.828427 87.828427) (mid 114 85) (end 116.828427 83.828427) (stroke (width 0.1) (type default)) (layer "Edge.Cuts"))
 (gr_arc (start 116.828427 106.171573) (mid 114 105) (end 112.828427 102.171573) (stroke (width 0.1) (type default)) (layer "Edge.Cuts"))
 (gr_arc (start 125.171573 83.828427) (mid 128 85) (end 129.171573 87.828427) (stroke (width 0.1) (type default)) (layer "Edge.Cuts"))
 (gr_line (start 129.171573 87.828427) (end 129 102) (stroke (width 0.1) (type default)) (layer "Edge.Cuts"))
 (gr_arc (start 129 102) (mid 127.828427 104.828427) (end 125 106) (stroke (width 0.1) (type default)) (layer "Edge.Cuts"))
 (gr_line (start 116.828427 106.171573) (end 125 106) (stroke (width 0.1) (type default)) (layer "Edge.Cuts"))
 (segment (start 115.24 96.52) (end 115.24 97.76) (width 0.25) (layer "F.Cu") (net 1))
 (segment (start 115.24 97.76) (end 114 99) (width 0.25) (layer "F.Cu") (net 1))
 (via (at 114 99) (size 0.8) (drill 0.4) (layers "F.Cu" "B.Cu") (free) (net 1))
 (segment (start 118.86 96.52) (end 119.38 96) (width 0.25) (layer "F.Cu") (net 2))
 (segment (start 116.84 96.52) (end 118.86 96.52) (width 0.25) (layer "F.Cu") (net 2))
 (segment (start 122 92) (end 122 89) (width 0.25) (layer "F.Cu") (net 4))
 (segment (start 122 89) (end 123 88) (width 0.25) (layer "F.Cu") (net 4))
 (segment (start 121.205 92.795) (end 122 92) (width 0.25) (layer "F.Cu") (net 4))
 (segment (start 123 88) (end 125 88) (width 0.25) (layer "F.Cu") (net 4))
 (segment (start 121.205 96) (end 121.205 92.795) (width 0.25) (layer "F.Cu") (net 4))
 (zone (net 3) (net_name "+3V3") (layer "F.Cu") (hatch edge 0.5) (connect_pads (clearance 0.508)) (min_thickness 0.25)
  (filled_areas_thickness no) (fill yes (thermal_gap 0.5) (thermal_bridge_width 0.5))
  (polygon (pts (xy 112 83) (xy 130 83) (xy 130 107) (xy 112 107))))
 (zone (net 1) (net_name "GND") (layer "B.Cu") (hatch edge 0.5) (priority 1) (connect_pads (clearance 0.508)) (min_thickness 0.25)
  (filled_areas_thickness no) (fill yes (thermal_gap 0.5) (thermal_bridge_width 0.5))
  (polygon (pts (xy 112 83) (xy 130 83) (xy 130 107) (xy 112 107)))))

